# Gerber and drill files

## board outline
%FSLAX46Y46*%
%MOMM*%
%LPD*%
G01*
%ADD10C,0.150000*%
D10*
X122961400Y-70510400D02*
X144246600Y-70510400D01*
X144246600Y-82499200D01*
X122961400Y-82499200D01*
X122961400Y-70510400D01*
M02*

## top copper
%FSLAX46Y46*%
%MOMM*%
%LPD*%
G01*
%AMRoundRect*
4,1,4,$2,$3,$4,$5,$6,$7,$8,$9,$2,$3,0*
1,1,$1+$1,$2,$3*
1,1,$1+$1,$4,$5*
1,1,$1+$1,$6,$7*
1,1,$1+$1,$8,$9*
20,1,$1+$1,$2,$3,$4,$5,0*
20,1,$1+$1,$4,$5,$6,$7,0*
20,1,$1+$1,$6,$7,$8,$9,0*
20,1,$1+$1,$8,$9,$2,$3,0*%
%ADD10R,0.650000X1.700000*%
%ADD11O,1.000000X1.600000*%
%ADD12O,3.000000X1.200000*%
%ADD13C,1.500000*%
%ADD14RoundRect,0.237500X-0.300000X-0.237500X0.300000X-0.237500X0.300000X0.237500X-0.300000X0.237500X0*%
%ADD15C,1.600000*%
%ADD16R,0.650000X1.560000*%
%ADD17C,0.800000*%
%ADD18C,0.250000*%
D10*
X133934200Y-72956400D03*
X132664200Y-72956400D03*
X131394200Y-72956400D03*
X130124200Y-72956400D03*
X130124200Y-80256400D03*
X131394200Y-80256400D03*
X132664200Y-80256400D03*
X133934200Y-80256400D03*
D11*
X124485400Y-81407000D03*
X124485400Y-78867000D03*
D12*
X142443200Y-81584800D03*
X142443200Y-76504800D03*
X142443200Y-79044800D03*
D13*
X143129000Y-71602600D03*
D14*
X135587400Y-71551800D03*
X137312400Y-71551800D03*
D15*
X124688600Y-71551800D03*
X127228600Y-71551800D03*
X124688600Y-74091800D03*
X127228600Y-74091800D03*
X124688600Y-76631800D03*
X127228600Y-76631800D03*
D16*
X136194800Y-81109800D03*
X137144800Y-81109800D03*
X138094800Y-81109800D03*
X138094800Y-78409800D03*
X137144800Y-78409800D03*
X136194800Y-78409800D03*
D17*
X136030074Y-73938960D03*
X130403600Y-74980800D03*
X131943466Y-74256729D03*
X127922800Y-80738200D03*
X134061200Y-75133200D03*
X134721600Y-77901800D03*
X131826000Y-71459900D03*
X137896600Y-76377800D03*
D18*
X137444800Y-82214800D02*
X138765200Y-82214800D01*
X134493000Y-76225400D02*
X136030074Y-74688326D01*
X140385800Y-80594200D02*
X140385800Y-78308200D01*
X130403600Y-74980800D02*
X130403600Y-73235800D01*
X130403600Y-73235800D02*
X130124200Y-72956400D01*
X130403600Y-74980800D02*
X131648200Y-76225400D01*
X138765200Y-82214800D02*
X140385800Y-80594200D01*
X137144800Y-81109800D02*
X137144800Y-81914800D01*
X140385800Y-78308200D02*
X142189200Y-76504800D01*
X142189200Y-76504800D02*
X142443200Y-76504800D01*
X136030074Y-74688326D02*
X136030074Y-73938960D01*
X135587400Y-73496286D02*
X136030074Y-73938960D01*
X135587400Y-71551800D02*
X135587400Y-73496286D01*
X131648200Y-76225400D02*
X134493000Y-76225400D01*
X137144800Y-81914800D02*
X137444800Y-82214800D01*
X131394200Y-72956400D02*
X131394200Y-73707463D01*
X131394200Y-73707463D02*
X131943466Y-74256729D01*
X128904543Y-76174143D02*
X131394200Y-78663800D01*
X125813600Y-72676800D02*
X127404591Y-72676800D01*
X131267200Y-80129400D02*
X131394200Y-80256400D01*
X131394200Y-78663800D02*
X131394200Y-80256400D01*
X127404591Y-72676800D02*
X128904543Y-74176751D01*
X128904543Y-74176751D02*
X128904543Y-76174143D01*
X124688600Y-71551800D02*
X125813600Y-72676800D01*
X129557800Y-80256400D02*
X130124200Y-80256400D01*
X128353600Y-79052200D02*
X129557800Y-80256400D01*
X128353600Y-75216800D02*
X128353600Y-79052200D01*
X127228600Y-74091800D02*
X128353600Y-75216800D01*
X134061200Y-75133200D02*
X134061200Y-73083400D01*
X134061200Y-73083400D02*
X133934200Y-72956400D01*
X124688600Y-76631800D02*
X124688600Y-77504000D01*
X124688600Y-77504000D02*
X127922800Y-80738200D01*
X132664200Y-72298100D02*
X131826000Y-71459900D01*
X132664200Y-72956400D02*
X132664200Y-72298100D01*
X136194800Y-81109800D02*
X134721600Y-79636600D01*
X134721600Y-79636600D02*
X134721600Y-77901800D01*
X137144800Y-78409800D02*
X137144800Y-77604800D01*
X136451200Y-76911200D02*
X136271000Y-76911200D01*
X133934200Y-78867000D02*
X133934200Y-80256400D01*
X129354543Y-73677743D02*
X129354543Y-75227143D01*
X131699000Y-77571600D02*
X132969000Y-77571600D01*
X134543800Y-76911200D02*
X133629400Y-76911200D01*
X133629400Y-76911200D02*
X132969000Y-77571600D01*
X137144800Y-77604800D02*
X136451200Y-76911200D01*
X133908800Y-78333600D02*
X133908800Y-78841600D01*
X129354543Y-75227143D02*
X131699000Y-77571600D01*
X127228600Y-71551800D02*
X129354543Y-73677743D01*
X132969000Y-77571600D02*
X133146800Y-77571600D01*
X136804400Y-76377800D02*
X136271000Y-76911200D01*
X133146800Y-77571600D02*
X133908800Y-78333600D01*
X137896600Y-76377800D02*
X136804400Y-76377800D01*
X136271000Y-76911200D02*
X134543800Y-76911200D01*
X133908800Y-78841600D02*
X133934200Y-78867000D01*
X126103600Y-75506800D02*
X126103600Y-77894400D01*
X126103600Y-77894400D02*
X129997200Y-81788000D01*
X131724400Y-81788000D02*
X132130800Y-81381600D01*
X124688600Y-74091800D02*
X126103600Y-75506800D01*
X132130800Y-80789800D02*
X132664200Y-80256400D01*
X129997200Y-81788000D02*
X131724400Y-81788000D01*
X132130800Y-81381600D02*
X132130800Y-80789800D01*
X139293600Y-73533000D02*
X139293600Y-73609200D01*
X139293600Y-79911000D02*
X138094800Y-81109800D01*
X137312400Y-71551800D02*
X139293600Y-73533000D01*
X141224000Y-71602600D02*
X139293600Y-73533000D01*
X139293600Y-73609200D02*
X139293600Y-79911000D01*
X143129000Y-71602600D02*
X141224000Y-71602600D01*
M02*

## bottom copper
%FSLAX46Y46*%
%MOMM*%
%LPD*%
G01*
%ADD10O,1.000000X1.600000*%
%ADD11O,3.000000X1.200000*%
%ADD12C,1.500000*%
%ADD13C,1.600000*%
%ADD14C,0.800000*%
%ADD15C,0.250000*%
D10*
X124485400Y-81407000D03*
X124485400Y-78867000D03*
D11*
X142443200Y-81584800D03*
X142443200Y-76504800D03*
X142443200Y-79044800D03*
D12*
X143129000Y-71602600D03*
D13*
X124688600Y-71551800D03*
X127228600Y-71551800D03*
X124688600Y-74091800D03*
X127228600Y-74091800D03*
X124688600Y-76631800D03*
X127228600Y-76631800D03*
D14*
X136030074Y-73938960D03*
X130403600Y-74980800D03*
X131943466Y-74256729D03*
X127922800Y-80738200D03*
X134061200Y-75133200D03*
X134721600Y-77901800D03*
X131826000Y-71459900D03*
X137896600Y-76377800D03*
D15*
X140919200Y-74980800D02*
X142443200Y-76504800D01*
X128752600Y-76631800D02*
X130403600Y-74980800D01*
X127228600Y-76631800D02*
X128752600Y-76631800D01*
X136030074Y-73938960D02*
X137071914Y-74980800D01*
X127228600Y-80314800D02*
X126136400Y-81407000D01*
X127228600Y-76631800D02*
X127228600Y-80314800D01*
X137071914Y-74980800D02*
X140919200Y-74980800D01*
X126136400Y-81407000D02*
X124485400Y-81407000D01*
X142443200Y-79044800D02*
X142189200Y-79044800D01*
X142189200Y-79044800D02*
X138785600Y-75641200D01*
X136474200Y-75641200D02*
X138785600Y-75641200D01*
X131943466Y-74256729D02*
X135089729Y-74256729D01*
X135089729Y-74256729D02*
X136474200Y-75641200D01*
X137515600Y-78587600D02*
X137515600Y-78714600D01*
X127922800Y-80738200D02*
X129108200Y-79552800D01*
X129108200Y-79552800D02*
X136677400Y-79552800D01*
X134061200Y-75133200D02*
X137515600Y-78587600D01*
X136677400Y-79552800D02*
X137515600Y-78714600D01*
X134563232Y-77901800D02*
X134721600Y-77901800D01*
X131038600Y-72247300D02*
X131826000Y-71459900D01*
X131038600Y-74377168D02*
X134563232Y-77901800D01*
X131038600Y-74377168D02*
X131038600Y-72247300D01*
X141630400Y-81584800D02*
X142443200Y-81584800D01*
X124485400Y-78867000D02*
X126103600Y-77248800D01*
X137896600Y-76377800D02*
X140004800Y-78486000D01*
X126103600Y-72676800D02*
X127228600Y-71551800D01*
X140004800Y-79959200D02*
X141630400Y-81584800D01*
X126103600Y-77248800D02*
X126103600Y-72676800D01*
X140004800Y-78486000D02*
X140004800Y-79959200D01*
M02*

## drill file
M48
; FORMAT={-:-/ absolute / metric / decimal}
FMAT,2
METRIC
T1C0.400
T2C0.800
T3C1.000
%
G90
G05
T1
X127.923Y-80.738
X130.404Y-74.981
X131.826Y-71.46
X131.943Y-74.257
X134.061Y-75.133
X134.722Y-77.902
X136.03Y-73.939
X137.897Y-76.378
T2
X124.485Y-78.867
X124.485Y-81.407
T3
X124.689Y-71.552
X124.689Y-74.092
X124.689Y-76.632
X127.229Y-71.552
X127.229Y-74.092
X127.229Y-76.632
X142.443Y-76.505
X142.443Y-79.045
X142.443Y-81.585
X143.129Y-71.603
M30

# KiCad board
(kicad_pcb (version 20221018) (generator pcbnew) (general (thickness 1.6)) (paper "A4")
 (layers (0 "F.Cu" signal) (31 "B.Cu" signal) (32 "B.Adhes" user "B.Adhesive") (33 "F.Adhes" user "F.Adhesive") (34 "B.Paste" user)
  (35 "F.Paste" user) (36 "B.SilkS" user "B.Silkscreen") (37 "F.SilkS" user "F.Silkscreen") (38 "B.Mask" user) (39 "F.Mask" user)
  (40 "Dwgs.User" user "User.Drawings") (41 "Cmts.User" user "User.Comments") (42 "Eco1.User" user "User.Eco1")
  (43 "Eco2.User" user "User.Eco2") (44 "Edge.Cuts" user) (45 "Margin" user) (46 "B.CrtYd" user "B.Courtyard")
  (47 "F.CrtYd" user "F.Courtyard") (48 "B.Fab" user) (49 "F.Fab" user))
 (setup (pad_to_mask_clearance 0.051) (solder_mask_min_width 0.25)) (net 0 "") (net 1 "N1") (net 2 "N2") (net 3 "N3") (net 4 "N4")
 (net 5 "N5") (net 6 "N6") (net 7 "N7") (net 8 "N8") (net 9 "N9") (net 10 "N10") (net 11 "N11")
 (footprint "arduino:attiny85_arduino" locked (layer "F.Cu") (at 132.0292 76.6064 -90)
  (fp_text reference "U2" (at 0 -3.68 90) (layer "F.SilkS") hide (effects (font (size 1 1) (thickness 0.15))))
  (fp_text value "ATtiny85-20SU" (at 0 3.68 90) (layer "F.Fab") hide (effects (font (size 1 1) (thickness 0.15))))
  (pad "1" smd rect locked (at -3.65 -1.905 270) (size 1.7 0.65) (layers "F.Cu" "F.Paste" "F.Mask") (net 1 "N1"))
  (pad "2" smd rect locked (at -3.65 -0.635 270) (size 1.7 0.65) (layers "F.Cu" "F.Paste" "F.Mask") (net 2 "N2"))
  (pad "3" smd rect locked (at -3.65 0.635 270) (size 1.7 0.65) (layers "F.Cu" "F.Paste" "F.Mask") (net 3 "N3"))
  (pad "4" smd rect locked (at -3.65 1.905 270) (size 1.7 0.65) (layers "F.Cu" "F.Paste" "F.Mask") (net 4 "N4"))
  (pad "5" smd rect locked (at 3.65 1.905 270) (size 1.7 0.65) (layers "F.Cu" "F.Paste" "F.Mask") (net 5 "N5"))
  (pad "6" smd rect locked (at 3.65 0.635 270) (size 1.7 0.65) (layers "F.Cu" "F.Paste" "F.Mask") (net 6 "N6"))
  (pad "7" smd rect locked (at 3.65 -0.635 270) (size 1.7 0.65) (layers "F.Cu" "F.Paste" "F.Mask") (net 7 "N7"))
  (pad "8" smd rect locked (at 3.65 -1.905 270) (size 1.7 0.65) (layers "F.Cu" "F.Paste" "F.Mask") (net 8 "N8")))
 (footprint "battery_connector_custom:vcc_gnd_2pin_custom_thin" (layer "F.Cu") (at 124.4854 80.137 90)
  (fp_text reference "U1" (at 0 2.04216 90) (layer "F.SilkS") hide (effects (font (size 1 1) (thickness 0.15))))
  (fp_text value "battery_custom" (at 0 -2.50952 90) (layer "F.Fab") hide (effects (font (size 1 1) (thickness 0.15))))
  (pad "1" thru_hole oval (at -1.27 0 90) (size 1.6 1) (drill 0.8) (layers "*.Cu" "*.Mask") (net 4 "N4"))
  (pad "2" thru_hole oval (at 1.27 0 90) (size 1.6 1) (drill 0.8) (layers "*.Cu" "*.Mask") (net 8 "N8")))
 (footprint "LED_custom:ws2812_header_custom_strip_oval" (layer "F.Cu") (at 142.4432 79.0448 -90)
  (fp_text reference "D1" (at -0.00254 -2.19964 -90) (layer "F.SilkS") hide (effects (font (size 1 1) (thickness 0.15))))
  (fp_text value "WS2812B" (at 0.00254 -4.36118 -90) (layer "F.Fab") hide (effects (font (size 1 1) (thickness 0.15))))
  (pad "1" thru_hole oval (at 2.54 0 270) (size 1.2 3) (drill 1) (layers "*.Cu" "*.Mask") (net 8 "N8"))
  (pad "3" thru_hole oval (at -2.54 0 270) (size 1.2 3) (drill 1) (layers "*.Cu" "*.Mask") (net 4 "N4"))
  (pad "4" thru_hole oval (at 0 0 270) (size 1.2 3) (drill 1) (layers "*.Cu" "*.Mask") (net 3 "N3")))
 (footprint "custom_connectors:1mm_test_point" (layer "F.Cu") (at 143.129 71.61276)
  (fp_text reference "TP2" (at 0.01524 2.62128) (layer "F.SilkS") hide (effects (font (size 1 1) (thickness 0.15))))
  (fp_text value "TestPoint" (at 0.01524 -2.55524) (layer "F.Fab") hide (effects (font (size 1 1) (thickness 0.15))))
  (pad "1" thru_hole circle (at 0 -0.01016) (size 1.5 1.5) (drill 1) (layers "*.Cu" "*.Mask") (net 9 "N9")))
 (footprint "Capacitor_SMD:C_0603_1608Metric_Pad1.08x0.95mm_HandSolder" (layer "F.Cu") (at 136.4499 71.5518)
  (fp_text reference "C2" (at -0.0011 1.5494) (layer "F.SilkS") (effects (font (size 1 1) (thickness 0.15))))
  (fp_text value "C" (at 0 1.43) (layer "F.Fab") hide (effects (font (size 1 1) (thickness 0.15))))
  (pad "1" smd roundrect (at -0.8625 0) (size 1.075 0.95) (layers "F.Cu" "F.Paste" "F.Mask") (roundrect_rratio 0.25) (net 4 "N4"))
  (pad "2" smd roundrect (at 0.8625 0) (size 1.075 0.95) (layers "F.Cu" "F.Paste" "F.Mask") (roundrect_rratio 0.25) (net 9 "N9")))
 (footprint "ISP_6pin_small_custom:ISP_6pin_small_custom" (layer "F.Cu") (at 125.9586 74.0918 90)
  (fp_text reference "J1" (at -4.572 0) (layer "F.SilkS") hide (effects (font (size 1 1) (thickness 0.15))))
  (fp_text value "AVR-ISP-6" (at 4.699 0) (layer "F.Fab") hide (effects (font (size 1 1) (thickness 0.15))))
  (pad "1" thru_hole circle (at 2.54 -1.27 90) (size 1.6 1.6) (drill 1) (layers "*.Cu" "*.Mask") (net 6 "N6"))
  (pad "2" thru_hole circle (at 2.54 1.27 90) (size 1.6 1.6) (drill 1) (layers "*.Cu" "*.Mask") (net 8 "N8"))
  (pad "3" thru_hole circle (at 0 -1.27 90) (size 1.6 1.6) (drill 1) (layers "*.Cu" "*.Mask") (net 7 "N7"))
  (pad "4" thru_hole circle (at 0 1.27 90) (size 1.6 1.6) (drill 1) (layers "*.Cu" "*.Mask") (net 5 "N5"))
  (pad "5" thru_hole circle (at -2.54 -1.27 90) (size 1.6 1.6) (drill 1) (layers "*.Cu" "*.Mask") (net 1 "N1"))
  (pad "6" thru_hole circle (at -2.54 1.27 90) (size 1.6 1.6) (drill 1) (layers "*.Cu" "*.Mask") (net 4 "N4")))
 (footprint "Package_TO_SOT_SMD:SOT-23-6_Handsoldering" (layer "F.Cu") (at 137.1448 79.7598 90)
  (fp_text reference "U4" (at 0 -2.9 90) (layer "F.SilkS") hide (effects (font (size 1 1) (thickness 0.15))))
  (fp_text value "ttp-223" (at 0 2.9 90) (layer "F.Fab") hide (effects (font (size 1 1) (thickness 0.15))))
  (pad "1" smd rect (at -1.35 -0.95 90) (size 1.56 0.65) (layers "F.Cu" "F.Paste" "F.Mask") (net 2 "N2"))
  (pad "2" smd rect (at -1.35 0 90) (size 1.56 0.65) (layers "F.Cu" "F.Paste" "F.Mask") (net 4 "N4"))
  (pad "3" smd rect (at -1.35 0.95 90) (size 1.56 0.65) (layers "F.Cu" "F.Paste" "F.Mask") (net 9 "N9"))
  (pad "4" smd rect (at 1.35 0.95 90) (size 1.56 0.65) (layers "F.Cu" "F.Paste" "F.Mask") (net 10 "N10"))
  (pad "5" smd rect (at 1.35 0 90) (size 1.56 0.65) (layers "F.Cu" "F.Paste" "F.Mask") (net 8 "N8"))
  (pad "6" smd rect (at 1.35 -0.95 90) (size 1.56 0.65) (layers "F.Cu" "F.Paste" "F.Mask") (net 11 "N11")))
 (gr_rect (start 122.9614 70.5104) (end 144.2466 82.4992) (stroke (width 0.15) (type solid)) (fill none) (layer "Edge.Cuts"))
 (segment (start 137.4448 82.2148) (end 138.7652 82.2148) (width 0.25) (layer "F.Cu") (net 4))
 (segment (start 134.493 76.2254) (end 136.030074 74.688326) (width 0.25) (layer "F.Cu") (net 4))
 (segment (start 140.3858 80.5942) (end 140.3858 78.3082) (width 0.25) (layer "F.Cu") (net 4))
 (segment (start 130.4036 74.9808) (end 130.4036 73.2358) (width 0.25) (layer "F.Cu") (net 4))
 (segment (start 130.4036 73.2358) (end 130.1242 72.9564) (width 0.25) (layer "F.Cu") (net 4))
 (segment (start 130.4036 74.9808) (end 131.6482 76.2254) (width 0.25) (layer "F.Cu") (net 4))
 (segment (start 138.7652 82.2148) (end 140.3858 80.5942) (width 0.25) (layer "F.Cu") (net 4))
 (segment (start 137.1448 81.1098) (end 137.1448 81.9148) (width 0.25) (layer "F.Cu") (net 4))
 (segment (start 140.3858 78.3082) (end 142.1892 76.5048) (width 0.25) (layer "F.Cu") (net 4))
 (segment (start 142.1892 76.5048) (end 142.4432 76.5048) (width 0.25) (layer "F.Cu") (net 4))
 (segment (start 136.030074 74.688326) (end 136.030074 73.93896) (width 0.25) (layer "F.Cu") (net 4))
 (segment (start 135.5874 73.496286) (end 136.030074 73.93896) (width 0.25) (layer "F.Cu") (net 4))
 (segment (start 135.5874 71.5518) (end 135.5874 73.496286) (width 0.25) (layer "F.Cu") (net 4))
 (segment (start 131.6482 76.2254) (end 134.493 76.2254) (width 0.25) (layer "F.Cu") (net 4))
 (segment (start 137.1448 81.9148) (end 137.4448 82.2148) (width 0.25) (layer "F.Cu") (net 4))
 (via (at 136.030074 73.93896) (size 0.8) (drill 0.4) (layers "F.Cu" "B.Cu") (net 4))
 (via (at 130.4036 74.9808) (size 0.8) (drill 0.4) (layers "F.Cu" "B.Cu") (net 4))
 (segment (start 140.9192 74.9808) (end 142.4432 76.5048) (width 0.25) (layer "B.Cu") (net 4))
 (segment (start 128.7526 76.6318) (end 130.4036 74.9808) (width 0.25) (layer "B.Cu") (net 4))
 (segment (start 127.2286 76.6318) (end 128.7526 76.6318) (width 0.25) (layer "B.Cu") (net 4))
 (segment (start 136.030074 73.93896) (end 137.071914 74.9808) (width 0.25) (layer "B.Cu") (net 4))
 (segment (start 127.2286 80.3148) (end 126.1364 81.407) (width 0.25) (layer "B.Cu") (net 4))
 (segment (start 127.2286 76.6318) (end 127.2286 80.3148) (width 0.25) (layer "B.Cu") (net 4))
 (segment (start 137.071914 74.9808) (end 140.9192 74.9808) (width 0.25) (layer "B.Cu") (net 4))
 (segment (start 126.1364 81.407) (end 124.4854 81.407) (width 0.25) (layer "B.Cu") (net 4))
 (segment (start 131.3942 72.9564) (end 131.3942 73.707463) (width 0.25) (layer "F.Cu") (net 3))
 (segment (start 131.3942 73.707463) (end 131.943466 74.256729) (width 0.25) (layer "F.Cu") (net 3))
 (via (at 131.943466 74.256729) (size 0.8) (drill 0.4) (layers "F.Cu" "B.Cu") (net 3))
 (segment (start 142.4432 79.0448) (end 142.1892 79.0448) (width 0.25) (layer "B.Cu") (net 3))
 (segment (start 142.1892 79.0448) (end 138.7856 75.6412) (width 0.25) (layer "B.Cu") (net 3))
 (segment (start 136.4742 75.6412) (end 138.7856 75.6412) (width 0.25) (layer "B.Cu") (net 3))
 (segment (start 131.943466 74.256729) (end 135.089729 74.256729) (width 0.25) (layer "B.Cu") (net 3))
 (segment (start 135.089729 74.256729) (end 136.4742 75.6412) (width 0.25) (layer "B.Cu") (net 3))
 (segment (start 128.904543 76.174143) (end 131.3942 78.6638) (width 0.25) (layer "F.Cu") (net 6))
 (segment (start 125.8136 72.6768) (end 127.404591 72.6768) (width 0.25) (layer "F.Cu") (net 6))
 (segment (start 131.2672 80.1294) (end 131.3942 80.2564) (width 0.25) (layer "F.Cu") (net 6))
 (segment (start 131.3942 78.6638) (end 131.3942 80.2564) (width 0.25) (layer "F.Cu") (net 6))
 (segment (start 127.404591 72.6768) (end 128.904543 74.176751) (width 0.25) (layer "F.Cu") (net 6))
 (segment (start 128.904543 74.176751) (end 128.904543 76.174143) (width 0.25) (layer "F.Cu") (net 6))
 (segment (start 124.6886 71.5518) (end 125.8136 72.6768) (width 0.25) (layer "F.Cu") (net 6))
 (segment (start 129.5578 80.2564) (end 130.1242 80.2564) (width 0.25) (layer "F.Cu") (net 5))
 (segment (start 128.3536 79.0522) (end 129.5578 80.2564) (width 0.25) (layer "F.Cu") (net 5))
 (segment (start 128.3536 75.2168) (end 128.3536 79.0522) (width 0.25) (layer "F.Cu") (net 5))
 (segment (start 127.2286 74.0918) (end 128.3536 75.2168) (width 0.25) (layer "F.Cu") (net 5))
 (segment (start 134.0612 75.1332) (end 134.0612 73.0834) (width 0.25) (layer "F.Cu") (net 1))
 (segment (start 134.0612 73.0834) (end 133.9342 72.9564) (width 0.25) (layer "F.Cu") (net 1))
 (segment (start 124.6886 76.6318) (end 124.6886 77.504) (width 0.25) (layer "F.Cu") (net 1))
 (segment (start 124.6886 77.504) (end 127.9228 80.7382) (width 0.25) (layer "F.Cu") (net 1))
 (via (at 127.9228 80.7382) (size 0.8) (drill 0.4) (layers "F.Cu" "B.Cu") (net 1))
 (via (at 134.0612 75.1332) (size 0.8) (drill 0.4) (layers "F.Cu" "B.Cu") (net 1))
 (segment (start 137.5156 78.5876) (end 137.5156 78.7146) (width 0.25) (layer "B.Cu") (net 1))
 (segment (start 127.9228 80.7382) (end 129.1082 79.5528) (width 0.25) (layer "B.Cu") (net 1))
 (segment (start 129.1082 79.5528) (end 136.6774 79.5528) (width 0.25) (layer "B.Cu") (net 1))
 (segment (start 134.0612 75.1332) (end 137.5156 78.5876) (width 0.25) (layer "B.Cu") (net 1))
 (segment (start 136.6774 79.5528) (end 137.5156 78.7146) (width 0.25) (layer "B.Cu") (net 1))
 (segment (start 132.6642 72.2981) (end 131.826 71.4599) (width 0.25) (layer "F.Cu") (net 2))
 (segment (start 132.6642 72.9564) (end 132.6642 72.2981) (width 0.25) (layer "F.Cu") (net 2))
 (segment (start 136.1948 81.1098) (end 134.7216 79.6366) (width 0.25) (layer "F.Cu") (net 2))
 (segment (start 134.7216 79.6366) (end 134.7216 77.9018) (width 0.25) (layer "F.Cu") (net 2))
 (via (at 134.7216 77.9018) (size 0.8) (drill 0.4) (layers "F.Cu" "B.Cu") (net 2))
 (via (at 131.826 71.4599) (size 0.8) (drill 0.4) (layers "F.Cu" "B.Cu") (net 2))
 (segment (start 134.563232 77.9018) (end 134.7216 77.9018) (width 0.25) (layer "B.Cu") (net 2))
 (segment (start 131.0386 72.2473) (end 131.826 71.4599) (width 0.25) (layer "B.Cu") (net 2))
 (segment (start 131.0386 74.377168) (end 134.563232 77.9018) (width 0.25) (layer "B.Cu") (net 2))
 (segment (start 131.0386 74.377168) (end 131.0386 72.2473) (width 0.25) (layer "B.Cu") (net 2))
 (segment (start 137.1448 78.4098) (end 137.1448 77.6048) (width 0.25) (layer "F.Cu") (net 8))
 (segment (start 136.4512 76.9112) (end 136.271 76.9112) (width 0.25) (layer "F.Cu") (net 8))
 (segment (start 133.9342 78.867) (end 133.9342 80.2564) (width 0.25) (layer "F.Cu") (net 8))
 (segment (start 129.354543 73.677743) (end 129.354543 75.227143) (width 0.25) (layer "F.Cu") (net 8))
 (segment (start 131.699 77.5716) (end 132.969 77.5716) (width 0.25) (layer "F.Cu") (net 8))
 (segment (start 134.5438 76.9112) (end 133.6294 76.9112) (width 0.25) (layer "F.Cu") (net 8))
 (segment (start 133.6294 76.9112) (end 132.969 77.5716) (width 0.25) (layer "F.Cu") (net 8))
 (segment (start 137.1448 77.6048) (end 136.4512 76.9112) (width 0.25) (layer "F.Cu") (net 8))
 (segment (start 133.9088 78.3336) (end 133.9088 78.8416) (width 0.25) (layer "F.Cu") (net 8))
 (segment (start 129.354543 75.227143) (end 131.699 77.5716) (width 0.25) (layer "F.Cu") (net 8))
 (segment (start 127.2286 71.5518) (end 129.354543 73.677743) (width 0.25) (layer "F.Cu") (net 8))
 (segment (start 132.969 77.5716) (end 133.1468 77.5716) (width 0.25) (layer "F.Cu") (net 8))
 (segment (start 136.8044 76.3778) (end 136.271 76.9112) (width 0.25) (layer "F.Cu") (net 8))
 (segment (start 133.1468 77.5716) (end 133.9088 78.3336) (width 0.25) (layer "F.Cu") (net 8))
 (segment (start 137.8966 76.3778) (end 136.8044 76.3778) (width 0.25) (layer "F.Cu") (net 8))
 (segment (start 136.271 76.9112) (end 134.5438 76.9112) (width 0.25) (layer "F.Cu") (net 8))
 (segment (start 133.9088 78.8416) (end 133.9342 78.867) (width 0.25) (layer "F.Cu") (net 8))
 (via (at 137.8966 76.3778) (size 0.8) (drill 0.4) (layers "F.Cu" "B.Cu") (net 8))
 (segment (start 141.6304 81.5848) (end 142.4432 81.5848) (width 0.25) (layer "B.Cu") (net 8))
 (segment (start 124.4854 78.867) (end 126.1036 77.2488) (width 0.25) (layer "B.Cu") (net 8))
 (segment (start 137.8966 76.3778) (end 140.0048 78.486) (width 0.25) (layer "B.Cu") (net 8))
 (segment (start 126.1036 72.6768) (end 127.2286 71.5518) (width 0.25) (layer "B.Cu") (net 8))
 (segment (start 140.0048 79.9592) (end 141.6304 81.5848) (width 0.25) (layer "B.Cu") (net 8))
 (segment (start 126.1036 77.2488) (end 126.1036 72.6768) (width 0.25) (layer "B.Cu") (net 8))
 (segment (start 140.0048 78.486) (end 140.0048 79.9592) (width 0.25) (layer "B.Cu") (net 8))
 (segment (start 126.1036 75.5068) (end 126.1036 77.8944) (width 0.25) (layer "F.Cu") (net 7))
 (segment (start 126.1036 77.8944) (end 129.9972 81.788) (width 0.25) (layer "F.Cu") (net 7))
 (segment (start 131.7244 81.788) (end 132.1308 81.3816) (width 0.25) (layer "F.Cu") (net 7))
 (segment (start 124.6886 74.0918) (end 126.1036 75.5068) (width 0.25) (layer "F.Cu") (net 7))
 (segment (start 132.1308 80.7898) (end 132.6642 80.2564) (width 0.25) (layer "F.Cu") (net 7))
 (segment (start 129.9972 81.788) (end 131.7244 81.788) (width 0.25) (layer "F.Cu") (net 7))
 (segment (start 132.1308 81.3816) (end 132.1308 80.7898) (width 0.25) (layer "F.Cu") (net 7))
 (segment (start 139.2936 73.533) (end 139.2936 73.6092) (width 0.25) (layer "F.Cu") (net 9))
 (segment (start 139.2936 79.911) (end 138.0948 81.1098) (width 0.25) (layer "F.Cu") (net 9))
 (segment (start 137.3124 71.5518) (end 139.2936 73.533) (width 0.25) (layer "F.Cu") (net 9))
 (segment (start 141.224 71.6026) (end 139.2936 73.533) (width 0.25) (layer "F.Cu") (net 9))
 (segment (start 139.2936 73.6092) (end 139.2936 79.911) (width 0.25) (layer "F.Cu") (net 9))
 (segment (start 143.129 71.6026) (end 141.224 71.6026) (width 0.25) (layer "F.Cu") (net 9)))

